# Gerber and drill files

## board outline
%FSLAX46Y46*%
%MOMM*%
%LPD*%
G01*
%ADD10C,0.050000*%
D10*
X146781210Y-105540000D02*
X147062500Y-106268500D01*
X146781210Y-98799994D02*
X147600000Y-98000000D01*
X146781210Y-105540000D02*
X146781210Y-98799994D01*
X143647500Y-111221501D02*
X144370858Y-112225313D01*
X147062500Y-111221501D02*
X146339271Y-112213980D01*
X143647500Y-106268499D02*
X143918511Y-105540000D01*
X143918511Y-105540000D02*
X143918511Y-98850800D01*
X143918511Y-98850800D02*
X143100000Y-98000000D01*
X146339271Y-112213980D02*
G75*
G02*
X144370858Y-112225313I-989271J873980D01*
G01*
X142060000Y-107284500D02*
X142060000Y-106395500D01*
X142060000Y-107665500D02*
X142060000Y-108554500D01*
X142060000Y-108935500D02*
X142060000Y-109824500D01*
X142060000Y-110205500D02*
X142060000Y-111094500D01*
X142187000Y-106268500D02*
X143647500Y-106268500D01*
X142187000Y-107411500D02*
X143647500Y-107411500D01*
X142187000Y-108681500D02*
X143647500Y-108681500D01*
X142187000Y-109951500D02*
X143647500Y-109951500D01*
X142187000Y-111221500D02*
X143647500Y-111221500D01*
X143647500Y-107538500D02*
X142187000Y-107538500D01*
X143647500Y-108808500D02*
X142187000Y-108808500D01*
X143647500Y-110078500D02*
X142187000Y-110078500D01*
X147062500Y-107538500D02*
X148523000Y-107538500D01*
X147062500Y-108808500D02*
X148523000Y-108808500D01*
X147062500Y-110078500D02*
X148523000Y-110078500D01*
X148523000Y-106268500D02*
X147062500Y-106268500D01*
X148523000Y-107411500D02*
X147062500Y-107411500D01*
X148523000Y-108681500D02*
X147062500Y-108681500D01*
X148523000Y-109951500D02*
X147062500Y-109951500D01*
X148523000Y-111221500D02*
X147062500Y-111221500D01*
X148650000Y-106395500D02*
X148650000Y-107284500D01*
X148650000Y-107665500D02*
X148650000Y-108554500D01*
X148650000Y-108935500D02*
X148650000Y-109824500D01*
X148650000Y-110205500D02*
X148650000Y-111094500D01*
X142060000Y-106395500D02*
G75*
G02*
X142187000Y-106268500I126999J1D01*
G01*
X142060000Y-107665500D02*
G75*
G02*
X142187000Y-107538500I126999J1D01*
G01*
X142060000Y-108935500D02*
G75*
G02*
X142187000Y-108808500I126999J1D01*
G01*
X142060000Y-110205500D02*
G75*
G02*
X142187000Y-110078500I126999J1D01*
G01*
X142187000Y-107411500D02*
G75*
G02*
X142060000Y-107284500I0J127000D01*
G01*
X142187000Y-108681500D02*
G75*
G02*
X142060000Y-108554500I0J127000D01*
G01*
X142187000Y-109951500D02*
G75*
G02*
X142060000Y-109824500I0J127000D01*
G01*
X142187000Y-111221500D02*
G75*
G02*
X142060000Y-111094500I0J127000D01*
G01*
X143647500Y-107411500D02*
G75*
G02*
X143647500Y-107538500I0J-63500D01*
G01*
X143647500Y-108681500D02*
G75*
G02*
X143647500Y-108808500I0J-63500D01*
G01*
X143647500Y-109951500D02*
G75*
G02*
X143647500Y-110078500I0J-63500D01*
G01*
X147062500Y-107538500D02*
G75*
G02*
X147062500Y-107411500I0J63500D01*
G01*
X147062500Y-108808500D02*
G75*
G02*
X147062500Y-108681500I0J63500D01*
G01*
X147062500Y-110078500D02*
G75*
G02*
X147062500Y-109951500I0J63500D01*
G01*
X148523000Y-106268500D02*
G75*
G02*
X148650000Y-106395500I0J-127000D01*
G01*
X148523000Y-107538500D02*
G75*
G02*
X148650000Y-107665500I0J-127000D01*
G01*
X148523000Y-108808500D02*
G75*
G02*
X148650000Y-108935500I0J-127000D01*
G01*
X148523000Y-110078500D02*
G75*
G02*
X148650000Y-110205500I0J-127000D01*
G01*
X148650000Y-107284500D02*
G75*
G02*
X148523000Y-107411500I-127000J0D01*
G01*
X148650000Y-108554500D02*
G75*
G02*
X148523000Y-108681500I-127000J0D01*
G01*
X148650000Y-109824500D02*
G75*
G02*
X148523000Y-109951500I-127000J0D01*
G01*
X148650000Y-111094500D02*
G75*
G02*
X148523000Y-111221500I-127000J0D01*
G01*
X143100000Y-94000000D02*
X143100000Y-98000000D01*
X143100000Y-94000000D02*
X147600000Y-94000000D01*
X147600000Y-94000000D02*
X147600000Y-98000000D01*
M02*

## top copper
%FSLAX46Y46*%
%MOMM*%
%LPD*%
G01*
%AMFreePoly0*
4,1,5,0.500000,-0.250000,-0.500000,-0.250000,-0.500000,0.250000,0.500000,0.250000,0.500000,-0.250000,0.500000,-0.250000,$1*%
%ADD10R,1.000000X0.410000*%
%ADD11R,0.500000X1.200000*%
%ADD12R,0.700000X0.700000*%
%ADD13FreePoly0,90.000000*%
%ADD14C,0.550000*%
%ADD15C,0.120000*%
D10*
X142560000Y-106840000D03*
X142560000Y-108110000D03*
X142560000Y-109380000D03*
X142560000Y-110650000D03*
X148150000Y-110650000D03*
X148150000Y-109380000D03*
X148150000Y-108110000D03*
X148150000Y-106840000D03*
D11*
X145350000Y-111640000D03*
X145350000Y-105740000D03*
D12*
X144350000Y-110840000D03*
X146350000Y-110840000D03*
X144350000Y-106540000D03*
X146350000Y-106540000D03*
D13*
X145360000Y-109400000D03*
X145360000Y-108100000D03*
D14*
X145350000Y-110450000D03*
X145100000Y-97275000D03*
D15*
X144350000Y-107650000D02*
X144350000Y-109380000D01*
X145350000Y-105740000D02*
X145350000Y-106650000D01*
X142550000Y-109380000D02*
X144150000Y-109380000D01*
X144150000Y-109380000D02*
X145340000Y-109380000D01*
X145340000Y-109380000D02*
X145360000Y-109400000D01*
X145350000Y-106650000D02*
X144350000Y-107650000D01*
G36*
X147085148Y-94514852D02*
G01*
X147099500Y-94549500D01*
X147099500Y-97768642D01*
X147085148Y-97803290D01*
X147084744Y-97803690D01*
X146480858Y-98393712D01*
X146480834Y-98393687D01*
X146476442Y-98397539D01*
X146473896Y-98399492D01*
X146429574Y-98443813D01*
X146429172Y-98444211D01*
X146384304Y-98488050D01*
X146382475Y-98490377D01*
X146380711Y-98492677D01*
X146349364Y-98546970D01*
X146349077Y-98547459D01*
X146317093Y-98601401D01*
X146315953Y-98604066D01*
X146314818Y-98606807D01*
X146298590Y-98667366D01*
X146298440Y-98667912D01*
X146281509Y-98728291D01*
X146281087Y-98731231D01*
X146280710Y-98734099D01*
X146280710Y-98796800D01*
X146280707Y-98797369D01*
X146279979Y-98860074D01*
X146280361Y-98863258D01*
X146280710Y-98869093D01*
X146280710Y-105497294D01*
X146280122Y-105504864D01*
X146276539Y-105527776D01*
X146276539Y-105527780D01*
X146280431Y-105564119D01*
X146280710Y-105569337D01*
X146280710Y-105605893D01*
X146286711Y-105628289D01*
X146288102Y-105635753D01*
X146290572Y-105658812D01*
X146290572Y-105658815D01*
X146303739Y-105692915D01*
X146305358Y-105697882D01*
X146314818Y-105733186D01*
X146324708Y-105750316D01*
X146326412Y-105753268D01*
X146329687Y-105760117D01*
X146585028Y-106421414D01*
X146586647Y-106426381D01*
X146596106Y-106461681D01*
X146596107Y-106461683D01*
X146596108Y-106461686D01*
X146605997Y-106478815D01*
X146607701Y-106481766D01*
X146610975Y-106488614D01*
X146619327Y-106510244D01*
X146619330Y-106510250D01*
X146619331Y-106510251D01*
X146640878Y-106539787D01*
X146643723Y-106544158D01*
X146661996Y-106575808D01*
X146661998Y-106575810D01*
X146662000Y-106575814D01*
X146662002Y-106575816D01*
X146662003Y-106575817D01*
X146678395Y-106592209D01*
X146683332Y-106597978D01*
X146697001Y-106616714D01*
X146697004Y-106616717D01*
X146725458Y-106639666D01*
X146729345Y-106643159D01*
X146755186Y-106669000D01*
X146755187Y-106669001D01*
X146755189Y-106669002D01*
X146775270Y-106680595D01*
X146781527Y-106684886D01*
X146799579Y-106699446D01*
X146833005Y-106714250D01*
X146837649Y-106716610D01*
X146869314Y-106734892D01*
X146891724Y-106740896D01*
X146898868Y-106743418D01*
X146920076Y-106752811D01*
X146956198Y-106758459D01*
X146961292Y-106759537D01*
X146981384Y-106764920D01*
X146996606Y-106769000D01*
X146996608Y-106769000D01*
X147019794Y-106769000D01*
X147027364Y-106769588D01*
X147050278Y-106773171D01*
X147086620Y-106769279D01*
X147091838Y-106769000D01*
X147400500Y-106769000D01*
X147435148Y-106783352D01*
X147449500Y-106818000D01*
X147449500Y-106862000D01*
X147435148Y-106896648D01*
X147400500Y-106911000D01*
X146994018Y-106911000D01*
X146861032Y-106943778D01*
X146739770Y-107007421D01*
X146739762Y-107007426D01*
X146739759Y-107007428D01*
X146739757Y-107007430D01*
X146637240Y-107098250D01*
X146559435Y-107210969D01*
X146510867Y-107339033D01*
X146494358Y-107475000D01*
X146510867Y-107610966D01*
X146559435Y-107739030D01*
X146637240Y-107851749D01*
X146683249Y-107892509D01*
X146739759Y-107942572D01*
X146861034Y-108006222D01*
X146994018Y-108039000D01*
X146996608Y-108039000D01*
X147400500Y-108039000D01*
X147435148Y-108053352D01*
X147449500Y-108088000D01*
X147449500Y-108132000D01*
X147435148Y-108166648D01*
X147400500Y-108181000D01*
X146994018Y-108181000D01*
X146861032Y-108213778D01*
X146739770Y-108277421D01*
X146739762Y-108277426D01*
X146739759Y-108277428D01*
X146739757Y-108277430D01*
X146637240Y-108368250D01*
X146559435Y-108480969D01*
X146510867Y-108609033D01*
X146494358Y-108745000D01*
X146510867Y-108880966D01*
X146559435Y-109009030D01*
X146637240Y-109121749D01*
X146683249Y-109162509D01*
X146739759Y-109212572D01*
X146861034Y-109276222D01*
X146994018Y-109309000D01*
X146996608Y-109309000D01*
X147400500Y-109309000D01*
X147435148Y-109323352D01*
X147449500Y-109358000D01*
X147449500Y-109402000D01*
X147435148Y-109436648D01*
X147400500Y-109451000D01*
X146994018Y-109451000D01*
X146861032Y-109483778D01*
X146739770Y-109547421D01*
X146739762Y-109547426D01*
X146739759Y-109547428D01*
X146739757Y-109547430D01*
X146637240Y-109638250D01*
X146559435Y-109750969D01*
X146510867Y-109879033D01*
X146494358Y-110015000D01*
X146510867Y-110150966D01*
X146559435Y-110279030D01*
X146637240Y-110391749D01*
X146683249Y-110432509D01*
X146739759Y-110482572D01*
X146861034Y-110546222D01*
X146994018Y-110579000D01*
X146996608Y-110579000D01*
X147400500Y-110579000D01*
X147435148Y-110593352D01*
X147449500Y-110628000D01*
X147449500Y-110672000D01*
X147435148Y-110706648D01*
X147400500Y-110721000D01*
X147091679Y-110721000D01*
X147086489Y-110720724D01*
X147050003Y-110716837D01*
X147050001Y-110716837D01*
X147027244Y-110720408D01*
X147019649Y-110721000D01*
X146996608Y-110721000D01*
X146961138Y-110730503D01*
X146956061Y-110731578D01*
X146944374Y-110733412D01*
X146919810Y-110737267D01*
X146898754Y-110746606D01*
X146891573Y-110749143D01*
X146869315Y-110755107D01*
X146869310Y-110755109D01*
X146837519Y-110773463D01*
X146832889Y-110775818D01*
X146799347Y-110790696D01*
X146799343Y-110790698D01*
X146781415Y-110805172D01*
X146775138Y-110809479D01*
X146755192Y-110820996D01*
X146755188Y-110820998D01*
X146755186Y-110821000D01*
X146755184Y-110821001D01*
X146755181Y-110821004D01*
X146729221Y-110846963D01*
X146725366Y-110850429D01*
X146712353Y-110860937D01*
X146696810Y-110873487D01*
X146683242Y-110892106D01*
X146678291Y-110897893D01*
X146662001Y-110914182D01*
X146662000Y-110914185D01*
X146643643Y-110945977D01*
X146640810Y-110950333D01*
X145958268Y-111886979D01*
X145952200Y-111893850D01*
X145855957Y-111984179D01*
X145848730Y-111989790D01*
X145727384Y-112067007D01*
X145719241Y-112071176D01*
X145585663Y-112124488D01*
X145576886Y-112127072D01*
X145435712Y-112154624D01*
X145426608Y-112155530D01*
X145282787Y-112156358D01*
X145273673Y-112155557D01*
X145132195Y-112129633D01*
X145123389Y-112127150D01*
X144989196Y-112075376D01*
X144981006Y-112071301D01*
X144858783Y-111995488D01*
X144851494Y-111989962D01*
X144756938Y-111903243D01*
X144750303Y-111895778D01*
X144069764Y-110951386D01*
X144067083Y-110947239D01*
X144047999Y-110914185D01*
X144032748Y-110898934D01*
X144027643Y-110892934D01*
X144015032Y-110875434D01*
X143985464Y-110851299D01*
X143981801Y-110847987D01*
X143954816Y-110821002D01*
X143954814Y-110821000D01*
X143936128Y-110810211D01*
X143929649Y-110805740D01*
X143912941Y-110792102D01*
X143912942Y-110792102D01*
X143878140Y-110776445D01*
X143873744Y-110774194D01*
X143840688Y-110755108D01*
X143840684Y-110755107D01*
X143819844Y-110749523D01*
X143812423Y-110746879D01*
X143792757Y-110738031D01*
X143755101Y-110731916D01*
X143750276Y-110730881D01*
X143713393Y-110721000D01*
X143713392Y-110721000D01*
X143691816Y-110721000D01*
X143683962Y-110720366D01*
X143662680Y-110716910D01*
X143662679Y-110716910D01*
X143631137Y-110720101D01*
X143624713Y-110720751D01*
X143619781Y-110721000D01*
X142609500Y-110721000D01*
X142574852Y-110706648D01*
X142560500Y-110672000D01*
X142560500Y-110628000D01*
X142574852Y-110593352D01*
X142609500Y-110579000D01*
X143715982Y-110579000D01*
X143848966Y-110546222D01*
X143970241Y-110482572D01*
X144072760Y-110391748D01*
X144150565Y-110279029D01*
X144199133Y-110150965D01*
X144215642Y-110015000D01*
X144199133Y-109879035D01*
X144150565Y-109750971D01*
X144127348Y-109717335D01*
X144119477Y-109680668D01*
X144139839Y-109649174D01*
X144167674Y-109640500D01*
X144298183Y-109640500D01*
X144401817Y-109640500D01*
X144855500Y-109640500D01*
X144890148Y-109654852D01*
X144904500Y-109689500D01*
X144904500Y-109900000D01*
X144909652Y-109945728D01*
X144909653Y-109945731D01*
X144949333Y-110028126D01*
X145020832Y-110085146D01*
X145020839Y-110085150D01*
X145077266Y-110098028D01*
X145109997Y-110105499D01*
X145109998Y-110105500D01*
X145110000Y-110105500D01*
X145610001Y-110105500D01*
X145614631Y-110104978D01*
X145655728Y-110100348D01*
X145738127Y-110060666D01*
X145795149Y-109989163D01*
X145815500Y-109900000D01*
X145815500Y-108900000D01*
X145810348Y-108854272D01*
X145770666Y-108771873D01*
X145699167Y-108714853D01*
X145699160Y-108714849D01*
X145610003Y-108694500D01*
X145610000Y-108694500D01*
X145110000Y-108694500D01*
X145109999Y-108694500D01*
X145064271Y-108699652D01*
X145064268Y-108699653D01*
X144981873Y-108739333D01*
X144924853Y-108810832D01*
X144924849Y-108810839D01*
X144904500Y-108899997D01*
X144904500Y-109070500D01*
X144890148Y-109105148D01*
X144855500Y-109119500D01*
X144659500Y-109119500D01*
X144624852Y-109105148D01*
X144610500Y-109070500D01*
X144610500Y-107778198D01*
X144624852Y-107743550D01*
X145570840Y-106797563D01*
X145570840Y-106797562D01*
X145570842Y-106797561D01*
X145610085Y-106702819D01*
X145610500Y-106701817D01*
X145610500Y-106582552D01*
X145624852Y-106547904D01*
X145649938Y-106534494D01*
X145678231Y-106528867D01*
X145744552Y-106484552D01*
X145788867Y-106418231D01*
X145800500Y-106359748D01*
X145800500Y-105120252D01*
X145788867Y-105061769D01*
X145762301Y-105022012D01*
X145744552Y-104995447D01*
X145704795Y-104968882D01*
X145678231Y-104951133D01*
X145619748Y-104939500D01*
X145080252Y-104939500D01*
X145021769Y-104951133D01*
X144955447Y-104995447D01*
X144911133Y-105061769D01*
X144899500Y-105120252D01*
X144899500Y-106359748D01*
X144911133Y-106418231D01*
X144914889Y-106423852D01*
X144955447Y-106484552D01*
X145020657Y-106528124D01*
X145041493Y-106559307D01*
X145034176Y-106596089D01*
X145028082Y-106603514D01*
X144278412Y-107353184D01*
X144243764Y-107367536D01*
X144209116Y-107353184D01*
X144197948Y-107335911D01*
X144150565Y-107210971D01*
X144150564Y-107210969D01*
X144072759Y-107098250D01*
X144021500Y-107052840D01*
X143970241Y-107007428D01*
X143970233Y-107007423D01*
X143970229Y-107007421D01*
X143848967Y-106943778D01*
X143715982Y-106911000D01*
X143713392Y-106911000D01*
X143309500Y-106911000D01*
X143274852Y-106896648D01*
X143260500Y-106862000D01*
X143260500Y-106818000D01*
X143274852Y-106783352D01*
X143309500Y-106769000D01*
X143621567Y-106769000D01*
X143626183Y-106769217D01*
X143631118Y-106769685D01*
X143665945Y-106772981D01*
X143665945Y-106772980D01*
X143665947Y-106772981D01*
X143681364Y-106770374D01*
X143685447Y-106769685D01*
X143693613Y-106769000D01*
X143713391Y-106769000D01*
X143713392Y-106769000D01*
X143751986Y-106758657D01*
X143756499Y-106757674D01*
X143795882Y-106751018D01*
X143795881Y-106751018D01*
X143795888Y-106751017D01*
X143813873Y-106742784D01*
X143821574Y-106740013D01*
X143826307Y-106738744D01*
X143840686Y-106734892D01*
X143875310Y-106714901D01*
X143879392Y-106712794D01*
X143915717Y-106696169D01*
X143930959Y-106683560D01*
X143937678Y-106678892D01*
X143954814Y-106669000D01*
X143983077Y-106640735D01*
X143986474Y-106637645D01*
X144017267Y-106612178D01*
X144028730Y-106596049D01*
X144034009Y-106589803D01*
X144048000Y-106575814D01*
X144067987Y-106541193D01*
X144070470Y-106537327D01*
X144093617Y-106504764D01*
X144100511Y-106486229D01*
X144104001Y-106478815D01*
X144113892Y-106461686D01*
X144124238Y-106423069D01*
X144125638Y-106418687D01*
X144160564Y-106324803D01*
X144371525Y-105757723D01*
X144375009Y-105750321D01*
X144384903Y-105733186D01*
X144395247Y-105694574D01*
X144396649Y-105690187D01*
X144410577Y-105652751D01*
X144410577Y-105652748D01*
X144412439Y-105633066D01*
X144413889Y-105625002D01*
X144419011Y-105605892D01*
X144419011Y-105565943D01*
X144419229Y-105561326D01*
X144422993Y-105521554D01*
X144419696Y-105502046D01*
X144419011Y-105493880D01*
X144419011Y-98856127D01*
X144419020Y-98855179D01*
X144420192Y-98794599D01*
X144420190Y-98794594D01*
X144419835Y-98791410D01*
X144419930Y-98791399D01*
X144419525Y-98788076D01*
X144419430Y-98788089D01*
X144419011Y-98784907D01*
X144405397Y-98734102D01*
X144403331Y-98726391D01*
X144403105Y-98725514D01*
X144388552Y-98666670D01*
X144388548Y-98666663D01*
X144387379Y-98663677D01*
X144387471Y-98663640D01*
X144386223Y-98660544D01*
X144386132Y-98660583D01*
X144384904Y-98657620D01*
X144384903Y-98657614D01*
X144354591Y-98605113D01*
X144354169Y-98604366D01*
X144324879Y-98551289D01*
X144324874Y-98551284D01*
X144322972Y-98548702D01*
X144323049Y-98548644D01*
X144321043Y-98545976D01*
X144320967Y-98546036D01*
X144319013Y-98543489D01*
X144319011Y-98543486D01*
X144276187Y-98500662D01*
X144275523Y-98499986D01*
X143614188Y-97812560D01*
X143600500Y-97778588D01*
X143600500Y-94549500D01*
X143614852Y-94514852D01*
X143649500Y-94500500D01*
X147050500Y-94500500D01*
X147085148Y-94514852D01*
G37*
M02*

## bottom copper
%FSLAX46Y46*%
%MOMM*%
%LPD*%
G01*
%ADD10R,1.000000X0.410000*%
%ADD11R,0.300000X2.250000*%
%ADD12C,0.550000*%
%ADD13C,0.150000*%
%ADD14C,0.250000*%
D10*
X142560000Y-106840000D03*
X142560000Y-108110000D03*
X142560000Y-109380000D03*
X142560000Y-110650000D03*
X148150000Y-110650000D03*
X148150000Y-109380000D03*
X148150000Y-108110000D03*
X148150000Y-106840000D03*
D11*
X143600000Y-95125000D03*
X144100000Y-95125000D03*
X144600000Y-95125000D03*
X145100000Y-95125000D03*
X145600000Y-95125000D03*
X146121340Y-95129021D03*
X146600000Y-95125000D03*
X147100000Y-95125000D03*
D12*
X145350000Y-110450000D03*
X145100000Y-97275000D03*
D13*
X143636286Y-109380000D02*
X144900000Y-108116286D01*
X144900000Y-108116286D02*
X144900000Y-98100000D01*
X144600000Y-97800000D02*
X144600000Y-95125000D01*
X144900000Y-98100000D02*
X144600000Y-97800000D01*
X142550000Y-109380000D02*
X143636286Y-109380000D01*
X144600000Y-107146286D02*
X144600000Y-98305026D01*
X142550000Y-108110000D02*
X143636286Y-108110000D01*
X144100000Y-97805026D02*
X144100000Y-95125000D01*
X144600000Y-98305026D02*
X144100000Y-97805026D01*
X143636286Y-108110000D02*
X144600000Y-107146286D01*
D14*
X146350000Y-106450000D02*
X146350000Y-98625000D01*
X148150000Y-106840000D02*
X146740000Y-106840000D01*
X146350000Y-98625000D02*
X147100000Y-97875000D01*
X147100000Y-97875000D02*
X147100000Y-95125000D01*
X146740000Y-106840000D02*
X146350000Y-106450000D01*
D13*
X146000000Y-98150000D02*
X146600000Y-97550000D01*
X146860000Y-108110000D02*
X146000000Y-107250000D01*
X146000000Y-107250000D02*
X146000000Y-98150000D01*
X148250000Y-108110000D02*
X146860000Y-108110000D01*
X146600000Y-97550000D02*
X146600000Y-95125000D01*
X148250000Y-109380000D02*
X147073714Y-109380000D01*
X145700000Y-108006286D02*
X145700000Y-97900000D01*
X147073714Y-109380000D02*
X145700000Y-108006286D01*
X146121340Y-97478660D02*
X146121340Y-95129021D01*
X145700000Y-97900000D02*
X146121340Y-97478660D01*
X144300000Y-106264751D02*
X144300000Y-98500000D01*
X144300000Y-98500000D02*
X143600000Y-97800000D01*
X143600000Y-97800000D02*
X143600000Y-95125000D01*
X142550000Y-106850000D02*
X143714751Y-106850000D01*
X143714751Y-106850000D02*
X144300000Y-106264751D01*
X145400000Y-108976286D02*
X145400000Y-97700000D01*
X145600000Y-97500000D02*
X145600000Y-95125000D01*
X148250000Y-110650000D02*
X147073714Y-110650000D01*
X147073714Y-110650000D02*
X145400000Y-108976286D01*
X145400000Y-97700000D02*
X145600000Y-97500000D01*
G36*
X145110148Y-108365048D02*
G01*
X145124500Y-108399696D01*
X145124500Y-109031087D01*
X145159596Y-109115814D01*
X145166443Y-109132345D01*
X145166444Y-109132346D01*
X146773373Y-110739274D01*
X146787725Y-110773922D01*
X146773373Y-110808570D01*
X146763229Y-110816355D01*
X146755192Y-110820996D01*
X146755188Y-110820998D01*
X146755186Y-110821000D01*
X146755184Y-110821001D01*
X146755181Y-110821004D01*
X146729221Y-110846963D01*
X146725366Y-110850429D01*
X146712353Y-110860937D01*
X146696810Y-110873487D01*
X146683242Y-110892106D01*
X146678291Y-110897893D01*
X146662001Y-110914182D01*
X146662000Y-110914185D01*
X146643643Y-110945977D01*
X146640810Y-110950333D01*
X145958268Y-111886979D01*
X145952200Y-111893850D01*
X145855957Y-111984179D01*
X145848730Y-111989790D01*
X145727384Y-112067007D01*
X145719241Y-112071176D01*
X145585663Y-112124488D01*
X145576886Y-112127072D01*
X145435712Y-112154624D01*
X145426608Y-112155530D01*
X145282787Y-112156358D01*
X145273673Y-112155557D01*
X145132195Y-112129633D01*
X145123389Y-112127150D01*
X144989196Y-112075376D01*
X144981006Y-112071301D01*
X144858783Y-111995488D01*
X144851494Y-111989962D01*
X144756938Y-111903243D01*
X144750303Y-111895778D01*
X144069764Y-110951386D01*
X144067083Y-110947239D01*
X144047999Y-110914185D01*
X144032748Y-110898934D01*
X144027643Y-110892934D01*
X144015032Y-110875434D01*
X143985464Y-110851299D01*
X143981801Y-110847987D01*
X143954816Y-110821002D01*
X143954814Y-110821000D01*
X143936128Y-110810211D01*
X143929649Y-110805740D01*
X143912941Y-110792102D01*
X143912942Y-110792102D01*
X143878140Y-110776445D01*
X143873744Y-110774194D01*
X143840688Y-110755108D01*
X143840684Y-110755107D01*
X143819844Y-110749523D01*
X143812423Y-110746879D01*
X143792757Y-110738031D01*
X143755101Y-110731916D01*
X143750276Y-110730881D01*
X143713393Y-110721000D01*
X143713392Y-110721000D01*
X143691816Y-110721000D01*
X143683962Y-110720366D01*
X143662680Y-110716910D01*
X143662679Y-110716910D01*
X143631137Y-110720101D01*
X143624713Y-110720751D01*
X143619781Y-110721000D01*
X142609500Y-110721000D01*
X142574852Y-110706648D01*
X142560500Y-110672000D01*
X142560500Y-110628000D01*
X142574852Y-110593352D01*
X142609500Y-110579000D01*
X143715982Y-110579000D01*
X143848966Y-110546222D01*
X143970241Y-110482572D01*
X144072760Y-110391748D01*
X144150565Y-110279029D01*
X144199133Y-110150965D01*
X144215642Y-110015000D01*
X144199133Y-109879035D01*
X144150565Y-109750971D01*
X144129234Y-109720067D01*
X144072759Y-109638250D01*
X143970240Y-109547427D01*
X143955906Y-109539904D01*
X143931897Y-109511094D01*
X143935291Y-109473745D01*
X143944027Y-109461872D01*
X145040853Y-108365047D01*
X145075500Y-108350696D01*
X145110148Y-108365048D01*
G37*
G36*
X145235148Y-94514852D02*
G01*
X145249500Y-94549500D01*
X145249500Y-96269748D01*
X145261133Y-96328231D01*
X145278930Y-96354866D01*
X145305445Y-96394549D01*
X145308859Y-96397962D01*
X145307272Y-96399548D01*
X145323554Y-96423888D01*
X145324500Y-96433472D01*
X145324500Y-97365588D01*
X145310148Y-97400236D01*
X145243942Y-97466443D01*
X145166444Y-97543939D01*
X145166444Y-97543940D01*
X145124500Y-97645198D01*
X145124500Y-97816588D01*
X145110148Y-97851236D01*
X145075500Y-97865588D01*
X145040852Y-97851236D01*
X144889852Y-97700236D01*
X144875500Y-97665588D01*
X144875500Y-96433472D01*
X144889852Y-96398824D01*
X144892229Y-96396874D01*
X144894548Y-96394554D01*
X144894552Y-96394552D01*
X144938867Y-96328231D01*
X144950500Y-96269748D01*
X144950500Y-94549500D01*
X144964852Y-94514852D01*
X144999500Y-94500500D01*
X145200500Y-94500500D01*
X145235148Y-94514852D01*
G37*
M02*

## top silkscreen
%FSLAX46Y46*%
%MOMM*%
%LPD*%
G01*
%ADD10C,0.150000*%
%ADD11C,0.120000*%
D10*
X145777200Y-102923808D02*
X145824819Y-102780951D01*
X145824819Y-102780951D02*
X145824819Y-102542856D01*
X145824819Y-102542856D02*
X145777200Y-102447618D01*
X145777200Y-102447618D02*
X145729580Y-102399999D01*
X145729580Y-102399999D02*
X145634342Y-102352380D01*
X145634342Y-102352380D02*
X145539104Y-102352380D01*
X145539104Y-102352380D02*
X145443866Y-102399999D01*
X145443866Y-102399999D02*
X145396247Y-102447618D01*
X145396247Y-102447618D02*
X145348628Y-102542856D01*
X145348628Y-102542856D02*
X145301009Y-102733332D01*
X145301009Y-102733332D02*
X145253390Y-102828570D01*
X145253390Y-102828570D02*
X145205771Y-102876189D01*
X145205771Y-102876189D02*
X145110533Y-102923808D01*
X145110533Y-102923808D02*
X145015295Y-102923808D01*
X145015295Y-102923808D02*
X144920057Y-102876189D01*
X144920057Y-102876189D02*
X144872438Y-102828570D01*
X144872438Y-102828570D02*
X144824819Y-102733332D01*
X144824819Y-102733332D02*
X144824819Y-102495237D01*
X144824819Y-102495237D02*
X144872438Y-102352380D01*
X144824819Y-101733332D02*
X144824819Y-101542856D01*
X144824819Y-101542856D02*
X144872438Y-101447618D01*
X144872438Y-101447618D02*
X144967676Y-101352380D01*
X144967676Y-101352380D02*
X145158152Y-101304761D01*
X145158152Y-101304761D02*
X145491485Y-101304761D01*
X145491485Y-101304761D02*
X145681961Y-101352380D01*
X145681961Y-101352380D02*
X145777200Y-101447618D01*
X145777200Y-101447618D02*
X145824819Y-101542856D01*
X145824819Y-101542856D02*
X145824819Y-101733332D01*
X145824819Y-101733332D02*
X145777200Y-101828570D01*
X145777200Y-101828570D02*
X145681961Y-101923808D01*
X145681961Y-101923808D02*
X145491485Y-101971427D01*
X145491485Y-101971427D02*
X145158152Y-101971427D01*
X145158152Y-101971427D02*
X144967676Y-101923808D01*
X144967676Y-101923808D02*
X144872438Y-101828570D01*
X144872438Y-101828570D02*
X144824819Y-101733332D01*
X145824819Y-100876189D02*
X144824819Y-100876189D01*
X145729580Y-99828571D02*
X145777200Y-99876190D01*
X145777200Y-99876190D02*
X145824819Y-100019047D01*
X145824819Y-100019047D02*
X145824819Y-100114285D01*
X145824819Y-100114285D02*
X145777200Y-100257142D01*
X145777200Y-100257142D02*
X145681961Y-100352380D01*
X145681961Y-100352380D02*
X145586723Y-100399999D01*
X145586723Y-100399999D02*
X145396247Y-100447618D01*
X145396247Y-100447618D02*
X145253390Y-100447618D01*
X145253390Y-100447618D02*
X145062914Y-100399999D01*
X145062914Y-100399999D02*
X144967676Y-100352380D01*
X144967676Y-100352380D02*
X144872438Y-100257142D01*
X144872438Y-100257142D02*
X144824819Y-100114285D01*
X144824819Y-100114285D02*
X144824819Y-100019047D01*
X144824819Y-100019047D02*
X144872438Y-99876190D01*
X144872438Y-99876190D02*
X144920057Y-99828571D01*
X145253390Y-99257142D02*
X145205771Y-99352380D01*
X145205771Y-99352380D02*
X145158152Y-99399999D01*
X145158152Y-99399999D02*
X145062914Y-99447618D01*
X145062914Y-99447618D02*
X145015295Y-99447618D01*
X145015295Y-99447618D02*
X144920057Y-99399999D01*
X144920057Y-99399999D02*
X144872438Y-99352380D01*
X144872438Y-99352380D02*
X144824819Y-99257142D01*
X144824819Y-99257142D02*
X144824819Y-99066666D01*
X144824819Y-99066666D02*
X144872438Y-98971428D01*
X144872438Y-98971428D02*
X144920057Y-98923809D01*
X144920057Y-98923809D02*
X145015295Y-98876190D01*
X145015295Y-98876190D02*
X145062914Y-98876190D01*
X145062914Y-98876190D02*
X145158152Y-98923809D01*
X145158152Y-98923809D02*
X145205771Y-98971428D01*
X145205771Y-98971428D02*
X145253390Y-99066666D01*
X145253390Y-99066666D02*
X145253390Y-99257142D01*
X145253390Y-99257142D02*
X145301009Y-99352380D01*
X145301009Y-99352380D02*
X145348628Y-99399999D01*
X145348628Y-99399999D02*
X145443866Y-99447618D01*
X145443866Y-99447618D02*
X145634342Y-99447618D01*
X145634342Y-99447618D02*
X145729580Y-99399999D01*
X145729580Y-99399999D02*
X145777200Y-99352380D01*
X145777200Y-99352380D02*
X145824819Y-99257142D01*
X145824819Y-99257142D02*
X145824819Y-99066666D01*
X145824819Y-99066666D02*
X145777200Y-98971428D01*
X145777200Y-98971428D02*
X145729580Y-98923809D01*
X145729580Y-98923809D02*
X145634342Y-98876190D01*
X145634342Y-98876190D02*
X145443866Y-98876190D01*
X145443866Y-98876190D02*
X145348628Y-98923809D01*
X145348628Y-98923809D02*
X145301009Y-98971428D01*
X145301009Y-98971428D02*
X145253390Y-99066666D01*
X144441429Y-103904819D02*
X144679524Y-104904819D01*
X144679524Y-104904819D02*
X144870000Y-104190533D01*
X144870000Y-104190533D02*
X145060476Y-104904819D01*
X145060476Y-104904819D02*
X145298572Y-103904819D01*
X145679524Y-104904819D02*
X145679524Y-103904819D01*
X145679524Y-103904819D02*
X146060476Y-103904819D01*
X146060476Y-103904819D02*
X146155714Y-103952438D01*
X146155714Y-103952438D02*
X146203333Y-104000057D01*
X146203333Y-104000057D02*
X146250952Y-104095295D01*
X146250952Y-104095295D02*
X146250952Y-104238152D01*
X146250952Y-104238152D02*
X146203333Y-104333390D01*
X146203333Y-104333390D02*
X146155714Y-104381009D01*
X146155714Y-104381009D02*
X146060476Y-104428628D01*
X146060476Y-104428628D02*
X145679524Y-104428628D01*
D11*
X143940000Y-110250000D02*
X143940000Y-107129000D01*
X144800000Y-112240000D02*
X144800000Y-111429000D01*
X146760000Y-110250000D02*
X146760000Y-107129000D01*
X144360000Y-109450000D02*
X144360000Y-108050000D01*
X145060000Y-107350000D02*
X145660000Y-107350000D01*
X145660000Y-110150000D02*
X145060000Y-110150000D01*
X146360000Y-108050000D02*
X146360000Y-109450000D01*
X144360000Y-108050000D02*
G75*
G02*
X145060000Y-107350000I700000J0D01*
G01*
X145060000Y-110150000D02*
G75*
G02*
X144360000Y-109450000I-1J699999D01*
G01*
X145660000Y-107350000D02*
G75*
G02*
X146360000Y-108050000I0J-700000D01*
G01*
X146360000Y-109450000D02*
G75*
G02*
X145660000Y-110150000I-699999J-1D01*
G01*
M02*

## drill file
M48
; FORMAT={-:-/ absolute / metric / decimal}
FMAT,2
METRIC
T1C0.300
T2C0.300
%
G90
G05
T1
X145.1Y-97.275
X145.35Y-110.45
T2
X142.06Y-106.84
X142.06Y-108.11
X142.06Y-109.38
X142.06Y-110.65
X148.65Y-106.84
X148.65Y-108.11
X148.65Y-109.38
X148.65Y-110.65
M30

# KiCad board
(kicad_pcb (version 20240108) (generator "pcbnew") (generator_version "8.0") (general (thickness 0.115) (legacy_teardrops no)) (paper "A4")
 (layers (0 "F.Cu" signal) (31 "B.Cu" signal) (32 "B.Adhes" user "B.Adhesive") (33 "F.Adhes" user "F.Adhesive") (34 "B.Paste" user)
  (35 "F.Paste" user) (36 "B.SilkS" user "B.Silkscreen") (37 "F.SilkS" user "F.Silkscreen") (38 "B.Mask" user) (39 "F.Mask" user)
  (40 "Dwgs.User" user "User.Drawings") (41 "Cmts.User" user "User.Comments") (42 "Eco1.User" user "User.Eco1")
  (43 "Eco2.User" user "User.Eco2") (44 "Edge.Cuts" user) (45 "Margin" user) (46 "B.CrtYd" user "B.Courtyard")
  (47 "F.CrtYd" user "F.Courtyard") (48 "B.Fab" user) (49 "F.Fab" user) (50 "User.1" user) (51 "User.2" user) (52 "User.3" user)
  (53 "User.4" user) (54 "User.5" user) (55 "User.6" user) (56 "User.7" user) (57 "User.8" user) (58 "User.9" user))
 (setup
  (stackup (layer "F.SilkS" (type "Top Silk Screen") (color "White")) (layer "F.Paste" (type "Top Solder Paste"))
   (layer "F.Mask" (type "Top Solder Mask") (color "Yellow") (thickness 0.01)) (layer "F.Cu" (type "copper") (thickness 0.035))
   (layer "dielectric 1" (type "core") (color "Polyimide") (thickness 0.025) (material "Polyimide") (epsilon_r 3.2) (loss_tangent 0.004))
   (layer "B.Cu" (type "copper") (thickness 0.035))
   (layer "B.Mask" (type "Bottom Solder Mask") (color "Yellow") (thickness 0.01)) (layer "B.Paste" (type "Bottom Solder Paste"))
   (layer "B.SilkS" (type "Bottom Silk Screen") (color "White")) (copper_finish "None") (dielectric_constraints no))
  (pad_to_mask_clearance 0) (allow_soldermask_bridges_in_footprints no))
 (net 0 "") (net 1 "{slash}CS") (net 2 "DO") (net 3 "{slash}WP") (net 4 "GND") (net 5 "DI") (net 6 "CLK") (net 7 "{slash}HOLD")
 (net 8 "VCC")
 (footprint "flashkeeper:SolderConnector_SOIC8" (layer "F.Cu") (at 142.06 106.84)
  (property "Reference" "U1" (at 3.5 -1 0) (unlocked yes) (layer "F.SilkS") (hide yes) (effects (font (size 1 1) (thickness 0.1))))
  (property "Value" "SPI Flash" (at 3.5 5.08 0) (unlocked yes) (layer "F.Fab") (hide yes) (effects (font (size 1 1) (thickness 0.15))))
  (fp_line (start 0 0.4445) (end 0 -0.4445) (stroke (width 0.05) (type default)) (layer "Edge.Cuts"))
  (fp_line (start 0 0.8255) (end 0 1.7145) (stroke (width 0.05) (type default)) (layer "Edge.Cuts"))
  (fp_line (start 0 2.0955) (end 0 2.9845) (stroke (width 0.05) (type default)) (layer "Edge.Cuts"))
  (fp_line (start 0 3.3655) (end 0 4.2545) (stroke (width 0.05) (type default)) (layer "Edge.Cuts"))
  (fp_line (start 0.127 -0.5715) (end 1.5875 -0.5715) (stroke (width 0.05) (type default)) (layer "Edge.Cuts"))
  (fp_line (start 0.127 0.5715) (end 1.5875 0.5715) (stroke (width 0.05) (type default)) (layer "Edge.Cuts"))
  (fp_line (start 0.127 1.8415) (end 1.5875 1.8415) (stroke (width 0.05) (type default)) (layer "Edge.Cuts"))
  (fp_line (start 0.127 3.1115) (end 1.5875 3.1115) (stroke (width 0.05) (type default)) (layer "Edge.Cuts"))
  (fp_line (start 0.127 4.3815) (end 1.5875 4.3815) (stroke (width 0.05) (type default)) (layer "Edge.Cuts"))
  (fp_line (start 1.5875 0.6985) (end 0.127 0.6985) (stroke (width 0.05) (type default)) (layer "Edge.Cuts"))
  (fp_line (start 1.5875 1.9685) (end 0.127 1.9685) (stroke (width 0.05) (type default)) (layer "Edge.Cuts"))
  (fp_line (start 1.5875 3.2385) (end 0.127 3.2385) (stroke (width 0.05) (type default)) (layer "Edge.Cuts"))
  (fp_line (start 5.0025 0.6985) (end 6.463 0.6985) (stroke (width 0.05) (type default)) (layer "Edge.Cuts"))
  (fp_line (start 5.0025 1.9685) (end 6.463 1.9685) (stroke (width 0.05) (type default)) (layer "Edge.Cuts"))
  (fp_line (start 5.0025 3.2385) (end 6.463 3.2385) (stroke (width 0.05) (type default)) (layer "Edge.Cuts"))
  (fp_line (start 6.463 -0.5715) (end 5.0025 -0.5715) (stroke (width 0.05) (type default)) (layer "Edge.Cuts"))
  (fp_line (start 6.463 0.5715) (end 5.0025 0.5715) (stroke (width 0.05) (type default)) (layer "Edge.Cuts"))
  (fp_line (start 6.463 1.8415) (end 5.0025 1.8415) (stroke (width 0.05) (type default)) (layer "Edge.Cuts"))
  (fp_line (start 6.463 3.1115) (end 5.0025 3.1115) (stroke (width 0.05) (type default)) (layer "Edge.Cuts"))
  (fp_line (start 6.463 4.3815) (end 5.0025 4.3815) (stroke (width 0.05) (type default)) (layer "Edge.Cuts"))
  (fp_line (start 6.59 -0.4445) (end 6.59 0.4445) (stroke (width 0.05) (type default)) (layer "Edge.Cuts"))
  (fp_line (start 6.59 0.8255) (end 6.59 1.7145) (stroke (width 0.05) (type default)) (layer "Edge.Cuts"))
  (fp_line (start 6.59 2.0955) (end 6.59 2.9845) (stroke (width 0.05) (type default)) (layer "Edge.Cuts"))
  (fp_line (start 6.59 3.3655) (end 6.59 4.2545) (stroke (width 0.05) (type default)) (layer "Edge.Cuts"))
  (fp_arc (start 0 -0.4445) (mid 0.037197 -0.534303) (end 0.127 -0.5715) (stroke (width 0.05) (type default)) (layer "Edge.Cuts"))
  (fp_arc (start 0 0.8255) (mid 0.037197 0.735697) (end 0.127 0.6985) (stroke (width 0.05) (type default)) (layer "Edge.Cuts"))
  (fp_arc (start 0 2.0955) (mid 0.037197 2.005697) (end 0.127 1.9685) (stroke (width 0.05) (type default)) (layer "Edge.Cuts"))
  (fp_arc (start 0 3.3655) (mid 0.037197 3.275697) (end 0.127 3.2385) (stroke (width 0.05) (type default)) (layer "Edge.Cuts"))
  (fp_arc (start 0.127 0.5715) (mid 0.037197 0.534303) (end 0 0.4445) (stroke (width 0.05) (type default)) (layer "Edge.Cuts"))
  (fp_arc (start 0.127 1.8415) (mid 0.037197 1.804303) (end 0 1.7145) (stroke (width 0.05) (type default)) (layer "Edge.Cuts"))
  (fp_arc (start 0.127 3.1115) (mid 0.037197 3.074303) (end 0 2.9845) (stroke (width 0.05) (type default)) (layer "Edge.Cuts"))
  (fp_arc (start 0.127 4.3815) (mid 0.037197 4.344303) (end 0 4.2545) (stroke (width 0.05) (type default)) (layer "Edge.Cuts"))
  (fp_arc (start 1.5875 0.5715) (mid 1.651 0.635) (end 1.5875 0.6985) (stroke (width 0.05) (type default)) (layer "Edge.Cuts"))
  (fp_arc (start 1.5875 1.8415) (mid 1.651 1.905) (end 1.5875 1.9685) (stroke (width 0.05) (type default)) (layer "Edge.Cuts"))
  (fp_arc (start 1.5875 3.1115) (mid 1.651 3.175) (end 1.5875 3.2385) (stroke (width 0.05) (type default)) (layer "Edge.Cuts"))
  (fp_arc (start 5.0025 0.6985) (mid 4.939 0.635) (end 5.0025 0.5715) (stroke (width 0.05) (type default)) (layer "Edge.Cuts"))
  (fp_arc (start 5.0025 1.9685) (mid 4.939 1.905) (end 5.0025 1.8415) (stroke (width 0.05) (type default)) (layer "Edge.Cuts"))
  (fp_arc (start 5.0025 3.2385) (mid 4.939 3.175) (end 5.0025 3.1115) (stroke (width 0.05) (type default)) (layer "Edge.Cuts"))
  (fp_arc (start 6.463 -0.5715) (mid 6.552803 -0.534303) (end 6.59 -0.4445) (stroke (width 0.05) (type default)) (layer "Edge.Cuts"))
  (fp_arc (start 6.463 0.6985) (mid 6.552803 0.735697) (end 6.59 0.8255) (stroke (width 0.05) (type default)) (layer "Edge.Cuts"))
  (fp_arc (start 6.463 1.9685) (mid 6.552803 2.005697) (end 6.59 2.0955) (stroke (width 0.05) (type default)) (layer "Edge.Cuts"))
  (fp_arc (start 6.463 3.2385) (mid 6.552803 3.275697) (end 6.59 3.3655) (stroke (width 0.05) (type default)) (layer "Edge.Cuts"))
  (fp_arc (start 6.59 0.4445) (mid 6.552803 0.534303) (end 6.463 0.5715) (stroke (width 0.05) (type default)) (layer "Edge.Cuts"))
  (fp_arc (start 6.59 1.7145) (mid 6.552803 1.804303) (end 6.463 1.8415) (stroke (width 0.05) (type default)) (layer "Edge.Cuts"))
  (fp_arc (start 6.59 2.9845) (mid 6.552803 3.074303) (end 6.463 3.1115) (stroke (width 0.05) (type default)) (layer "Edge.Cuts"))
  (fp_arc (start 6.59 4.2545) (mid 6.552803 4.344303) (end 6.463 4.3815) (stroke (width 0.05) (type default)) (layer "Edge.Cuts"))
  (pad "1" thru_hole rect (at 0 0) (size 1 0.41) (drill 0.3 (offset 0.5 0)) (layers "*.Cu" "*.Mask") (remove_unused_layers no)
   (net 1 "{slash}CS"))
  (pad "2" thru_hole rect (at 0 1.27) (size 1 0.41) (drill 0.3 (offset 0.5 0)) (layers "*.Cu" "*.Mask") (remove_unused_layers no)
   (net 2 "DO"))
  (pad "3" thru_hole rect (at 0 2.54) (size 1 0.41) (drill 0.3 (offset 0.5 0)) (layers "*.Cu" "*.Mask") (remove_unused_layers no)
   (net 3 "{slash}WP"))
  (pad "4" thru_hole rect (at 0 3.81) (size 1 0.41) (drill 0.3 (offset 0.5 0)) (layers "*.Cu" "*.Mask") (remove_unused_layers no)
   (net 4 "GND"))
  (pad "5" thru_hole rect (at 6.59 3.81 180) (size 1 0.41) (drill 0.3 (offset 0.5 0)) (layers "*.Cu" "*.Mask") (remove_unused_layers no)
   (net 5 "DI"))
  (pad "6" thru_hole rect (at 6.59 2.54 180) (size 1 0.41) (drill 0.3 (offset 0.5 0)) (layers "*.Cu" "*.Mask") (remove_unused_layers no)
   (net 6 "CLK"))
  (pad "7" thru_hole rect (at 6.59 1.27 180) (size 1 0.41) (drill 0.3 (offset 0.5 0)) (layers "*.Cu" "*.Mask") (remove_unused_layers no)
   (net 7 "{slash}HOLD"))
  (pad "8" thru_hole rect (at 6.59 0 180) (size 1 0.41) (drill 0.3 (offset 0.5 0)) (layers "*.Cu" "*.Mask") (remove_unused_layers no)
   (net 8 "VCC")))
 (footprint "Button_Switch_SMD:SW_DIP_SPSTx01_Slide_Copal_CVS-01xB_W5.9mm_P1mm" (layer "F.Cu") (at 145.35 108.69 90)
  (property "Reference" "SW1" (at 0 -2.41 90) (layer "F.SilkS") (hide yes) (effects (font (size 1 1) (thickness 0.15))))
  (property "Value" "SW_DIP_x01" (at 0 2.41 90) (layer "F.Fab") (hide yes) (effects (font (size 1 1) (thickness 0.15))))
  (fp_line (start -1.56 -1.41) (end 1.561 -1.41) (stroke (width 0.12) (type solid)) (layer "F.SilkS"))
  (fp_line (start -3.55 -0.55) (end -2.739 -0.55) (stroke (width 0.12) (type solid)) (layer "F.SilkS"))
  (fp_line (start -1.56 1.41) (end 1.561 1.41) (stroke (width 0.12) (type solid)) (layer "F.SilkS"))
  (pad "1" smd rect (at -2.95 0 90) (size 1.2 0.5) (layers "F.Cu" "F.Paste" "F.Mask") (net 4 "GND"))
  (pad "2" smd rect (at 2.95 0 90) (size 1.2 0.5) (layers "F.Cu" "F.Paste" "F.Mask") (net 3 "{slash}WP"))
  (pad "3" smd rect (at -2.15 -1 90) (size 0.7 0.7) (layers "F.Cu" "F.Paste" "F.Mask") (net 4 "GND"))
  (pad "3" smd rect (at -2.15 1 90) (size 0.7 0.7) (layers "F.Cu" "F.Paste" "F.Mask") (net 4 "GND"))
  (pad "3" smd rect (at 2.15 -1 90) (size 0.7 0.7) (layers "F.Cu" "F.Paste" "F.Mask") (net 4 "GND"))
  (pad "3" smd rect (at 2.15 1 90) (size 0.7 0.7) (layers "F.Cu" "F.Paste" "F.Mask") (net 4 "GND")))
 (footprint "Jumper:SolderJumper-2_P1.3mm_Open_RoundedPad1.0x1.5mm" (layer "F.Cu") (at 145.36 108.75 90)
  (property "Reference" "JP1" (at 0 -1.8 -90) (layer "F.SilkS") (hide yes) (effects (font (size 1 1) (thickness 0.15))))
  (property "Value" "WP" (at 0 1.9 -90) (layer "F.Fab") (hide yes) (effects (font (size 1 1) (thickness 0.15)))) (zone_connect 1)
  (fp_line (start -0.7 -1) (end 0.7 -1) (stroke (width 0.12) (type solid)) (layer "F.SilkS"))
  (fp_line (start 1.4 -0.3) (end 1.4 0.3) (stroke (width 0.12) (type solid)) (layer "F.SilkS"))
  (fp_line (start -1.4 0.3) (end -1.4 -0.3) (stroke (width 0.12) (type solid)) (layer "F.SilkS"))
  (fp_line (start 0.7 1) (end -0.7 1) (stroke (width 0.12) (type solid)) (layer "F.SilkS"))
  (fp_arc (start 0.7 -1) (mid 1.194975 -0.794975) (end 1.4 -0.3) (stroke (width 0.12) (type solid)) (layer "F.SilkS"))
  (fp_arc (start -1.4 -0.3) (mid -1.194975 -0.794975) (end -0.7 -1) (stroke (width 0.12) (type solid)) (layer "F.SilkS"))
  (fp_arc (start 1.4 0.3) (mid 1.194975 0.794975) (end 0.7 1) (stroke (width 0.12) (type solid)) (layer "F.SilkS"))
  (fp_arc (start -0.7 1) (mid -1.194975 0.794975) (end -1.4 0.3) (stroke (width 0.12) (type solid)) (layer "F.SilkS"))
  (pad "1" smd custom (at -0.65 0 90) (size 1 0.5) (layers "F.Cu" "F.Mask") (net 3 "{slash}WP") (zone_connect 2) (thermal_bridge_angle 45)
   (options (clearance outline) (anchor rect)) (primitives))
  (pad "2" smd custom (at 0.65 0 90) (size 1 0.5) (layers "F.Cu" "F.Mask") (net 4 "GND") (zone_connect 2) (thermal_bridge_angle 45)
   (options (clearance outline) (anchor rect)) (primitives)))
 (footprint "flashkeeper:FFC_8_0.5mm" (layer "F.Cu") (at 145.35 94)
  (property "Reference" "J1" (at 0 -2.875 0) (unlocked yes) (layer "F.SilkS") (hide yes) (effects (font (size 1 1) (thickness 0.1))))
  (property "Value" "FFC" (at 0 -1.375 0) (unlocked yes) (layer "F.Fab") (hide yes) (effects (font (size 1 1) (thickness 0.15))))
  (fp_line (start -2.25 0) (end -2.25 4) (stroke (width 0.05) (type default)) (layer "Edge.Cuts"))
  (fp_line (start -2.25 0) (end 2.25 0) (stroke (width 0.05) (type default)) (layer "Edge.Cuts"))
  (fp_line (start 2.25 0) (end 2.25 4) (stroke (width 0.05) (type default)) (layer "Edge.Cuts"))
  (pad "1" smd rect (at -1.75 1.125) (size 0.3 2.25) (layers "B.Cu" "B.Mask") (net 1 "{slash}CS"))
  (pad "2" smd rect (at -1.25 1.125) (size 0.3 2.25) (layers "B.Cu" "B.Mask") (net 2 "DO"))
  (pad "3" smd rect (at -0.75 1.125) (size 0.3 2.25) (layers "B.Cu" "B.Mask") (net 3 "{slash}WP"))
  (pad "4" smd rect (at -0.25 1.125) (size 0.3 2.25) (layers "B.Cu" "B.Mask") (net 4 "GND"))
  (pad "5" smd rect (at 0.25 1.125) (size 0.3 2.25) (layers "B.Cu" "B.Mask") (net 5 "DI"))
  (pad "6" smd rect (at 0.77134 1.129021) (size 0.3 2.25) (layers "B.Cu" "B.Mask") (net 6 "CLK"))
  (pad "7" smd rect (at 1.25 1.125) (size 0.3 2.25) (layers "B.Cu" "B.Mask") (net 7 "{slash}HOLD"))
  (pad "8" smd rect (at 1.75 1.125) (size 0.3 2.25) (layers "B.Cu" "B.Mask") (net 8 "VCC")))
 (gr_line (start 146.78121 105.54) (end 147.0625 106.2685) (stroke (width 0.05) (type default)) (layer "Edge.Cuts"))
 (gr_line (start 146.78121 98.799994) (end 147.6 98) (stroke (width 0.05) (type default)) (layer "Edge.Cuts"))
 (gr_line (start 146.78121 105.54) (end 146.78121 98.799994) (stroke (width 0.05) (type default)) (layer "Edge.Cuts"))
 (gr_line (start 143.6475 111.221501) (end 144.370858 112.225313) (stroke (width 0.05) (type default)) (layer "Edge.Cuts"))
 (gr_line (start 147.0625 111.221501) (end 146.339271 112.21398) (stroke (width 0.05) (type default)) (layer "Edge.Cuts"))
 (gr_line (start 143.6475 106.268499) (end 143.918511 105.54) (stroke (width 0.05) (type default)) (layer "Edge.Cuts"))
 (gr_line (start 143.918511 105.54) (end 143.918511 98.8508) (stroke (width 0.05) (type default)) (layer "Edge.Cuts"))
 (gr_line (start 143.918511 98.8508) (end 143.1 98) (stroke (width 0.05) (type default)) (layer "Edge.Cuts"))
 (gr_arc (start 146.339271 112.21398) (mid 145.3576 112.660015) (end 144.370858 112.225313) (stroke (width 0.05) (type default))
  (layer "Edge.Cuts"))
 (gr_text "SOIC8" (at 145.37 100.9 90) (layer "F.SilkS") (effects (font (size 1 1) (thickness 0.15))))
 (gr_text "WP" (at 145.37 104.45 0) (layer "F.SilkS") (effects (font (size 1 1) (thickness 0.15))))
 (segment (start 144.35 107.65) (end 144.35 109.38) (width 0.12) (layer "F.Cu") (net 3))
 (segment (start 145.35 105.74) (end 145.35 106.65) (width 0.12) (layer "F.Cu") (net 3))
 (segment (start 142.55 109.38) (end 144.15 109.38) (width 0.12) (layer "F.Cu") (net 3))
 (segment (start 144.15 109.38) (end 145.34 109.38) (width 0.12) (layer "F.Cu") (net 3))
 (segment (start 145.34 109.38) (end 145.36 109.4) (width 0.12) (layer "F.Cu") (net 3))
 (segment (start 145.35 106.65) (end 144.35 107.65) (width 0.12) (layer "F.Cu") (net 3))
 (segment (start 143.636286 109.38) (end 144.9 108.116286) (width 0.15) (layer "B.Cu") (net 3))
 (segment (start 144.9 108.116286) (end 144.9 98.1) (width 0.15) (layer "B.Cu") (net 3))
 (segment (start 144.6 97.8) (end 144.6 95.125) (width 0.15) (layer "B.Cu") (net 3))
 (segment (start 144.9 98.1) (end 144.6 97.8) (width 0.15) (layer "B.Cu") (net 3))
 (segment (start 142.55 109.38) (end 143.636286 109.38) (width 0.15) (layer "B.Cu") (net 3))
 (via (at 145.35 110.45) (size 0.55) (drill 0.3) (layers "F.Cu" "B.Cu") (free yes) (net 4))
 (via (at 145.1 97.275) (size 0.55) (drill 0.3) (layers "F.Cu" "B.Cu") (free yes) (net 4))
 (segment (start 144.6 107.146286) (end 144.6 98.305026) (width 0.15) (layer "B.Cu") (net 2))
 (segment (start 142.55 108.11) (end 143.636286 108.11) (width 0.15) (layer "B.Cu") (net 2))
 (segment (start 144.1 97.805026) (end 144.1 95.125) (width 0.15) (layer "B.Cu") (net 2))
 (segment (start 144.6 98.305026) (end 144.1 97.805026) (width 0.15) (layer "B.Cu") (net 2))
 (segment (start 143.636286 108.11) (end 144.6 107.146286) (width 0.15) (layer "B.Cu") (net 2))
 (segment (start 146.35 106.45) (end 146.35 98.625) (width 0.25) (layer "B.Cu") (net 8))
 (segment (start 148.15 106.84) (end 146.74 106.84) (width 0.25) (layer "B.Cu") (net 8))
 (segment (start 146.35 98.625) (end 147.1 97.875) (width 0.25) (layer "B.Cu") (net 8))
 (segment (start 147.1 97.875) (end 147.1 95.125) (width 0.25) (layer "B.Cu") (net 8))
 (segment (start 146.74 106.84) (end 146.35 106.45) (width 0.25) (layer "B.Cu") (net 8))
 (segment (start 146 98.15) (end 146.6 97.55) (width 0.15) (layer "B.Cu") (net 7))
 (segment (start 146.86 108.11) (end 146 107.25) (width 0.15) (layer "B.Cu") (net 7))
 (segment (start 146 107.25) (end 146 98.15) (width 0.15) (layer "B.Cu") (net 7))
 (segment (start 148.25 108.11) (end 146.86 108.11) (width 0.15) (layer "B.Cu") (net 7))
 (segment (start 146.6 97.55) (end 146.6 95.125) (width 0.15) (layer "B.Cu") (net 7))
 (segment (start 148.25 109.38) (end 147.073714 109.38) (width 0.15) (layer "B.Cu") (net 6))
 (segment (start 145.7 108.006286) (end 145.7 97.9) (width 0.15) (layer "B.Cu") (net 6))
 (segment (start 147.073714 109.38) (end 145.7 108.006286) (width 0.15) (layer "B.Cu") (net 6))
 (segment (start 146.12134 97.47866) (end 146.12134 95.129021) (width 0.15) (layer "B.Cu") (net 6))
 (segment (start 145.7 97.9) (end 146.12134 97.47866) (width 0.15) (layer "B.Cu") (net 6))
 (segment (start 144.3 106.264751) (end 144.3 98.5) (width 0.15) (layer "B.Cu") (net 1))
 (segment (start 144.3 98.5) (end 143.6 97.8) (width 0.15) (layer "B.Cu") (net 1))
 (segment (start 143.6 97.8) (end 143.6 95.125) (width 0.15) (layer "B.Cu") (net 1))
 (segment (start 142.55 106.85) (end 143.714751 106.85) (width 0.15) (layer "B.Cu") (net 1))
 (segment (start 143.714751 106.85) (end 144.3 106.264751) (width 0.15) (layer "B.Cu") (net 1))
 (segment (start 145.4 108.976286) (end 145.4 97.7) (width 0.15) (layer "B.Cu") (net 5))
 (segment (start 145.6 97.5) (end 145.6 95.125) (width 0.15) (layer "B.Cu") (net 5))
 (segment (start 148.25 110.65) (end 147.073714 110.65) (width 0.15) (layer "B.Cu") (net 5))
 (segment (start 147.073714 110.65) (end 145.4 108.976286) (width 0.15) (layer "B.Cu") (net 5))
 (segment (start 145.4 97.7) (end 145.6 97.5) (width 0.15) (layer "B.Cu") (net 5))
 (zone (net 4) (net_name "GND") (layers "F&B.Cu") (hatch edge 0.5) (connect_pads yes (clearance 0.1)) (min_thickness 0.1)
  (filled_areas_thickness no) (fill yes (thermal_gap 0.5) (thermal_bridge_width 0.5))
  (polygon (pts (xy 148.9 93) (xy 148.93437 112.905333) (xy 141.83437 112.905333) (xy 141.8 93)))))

